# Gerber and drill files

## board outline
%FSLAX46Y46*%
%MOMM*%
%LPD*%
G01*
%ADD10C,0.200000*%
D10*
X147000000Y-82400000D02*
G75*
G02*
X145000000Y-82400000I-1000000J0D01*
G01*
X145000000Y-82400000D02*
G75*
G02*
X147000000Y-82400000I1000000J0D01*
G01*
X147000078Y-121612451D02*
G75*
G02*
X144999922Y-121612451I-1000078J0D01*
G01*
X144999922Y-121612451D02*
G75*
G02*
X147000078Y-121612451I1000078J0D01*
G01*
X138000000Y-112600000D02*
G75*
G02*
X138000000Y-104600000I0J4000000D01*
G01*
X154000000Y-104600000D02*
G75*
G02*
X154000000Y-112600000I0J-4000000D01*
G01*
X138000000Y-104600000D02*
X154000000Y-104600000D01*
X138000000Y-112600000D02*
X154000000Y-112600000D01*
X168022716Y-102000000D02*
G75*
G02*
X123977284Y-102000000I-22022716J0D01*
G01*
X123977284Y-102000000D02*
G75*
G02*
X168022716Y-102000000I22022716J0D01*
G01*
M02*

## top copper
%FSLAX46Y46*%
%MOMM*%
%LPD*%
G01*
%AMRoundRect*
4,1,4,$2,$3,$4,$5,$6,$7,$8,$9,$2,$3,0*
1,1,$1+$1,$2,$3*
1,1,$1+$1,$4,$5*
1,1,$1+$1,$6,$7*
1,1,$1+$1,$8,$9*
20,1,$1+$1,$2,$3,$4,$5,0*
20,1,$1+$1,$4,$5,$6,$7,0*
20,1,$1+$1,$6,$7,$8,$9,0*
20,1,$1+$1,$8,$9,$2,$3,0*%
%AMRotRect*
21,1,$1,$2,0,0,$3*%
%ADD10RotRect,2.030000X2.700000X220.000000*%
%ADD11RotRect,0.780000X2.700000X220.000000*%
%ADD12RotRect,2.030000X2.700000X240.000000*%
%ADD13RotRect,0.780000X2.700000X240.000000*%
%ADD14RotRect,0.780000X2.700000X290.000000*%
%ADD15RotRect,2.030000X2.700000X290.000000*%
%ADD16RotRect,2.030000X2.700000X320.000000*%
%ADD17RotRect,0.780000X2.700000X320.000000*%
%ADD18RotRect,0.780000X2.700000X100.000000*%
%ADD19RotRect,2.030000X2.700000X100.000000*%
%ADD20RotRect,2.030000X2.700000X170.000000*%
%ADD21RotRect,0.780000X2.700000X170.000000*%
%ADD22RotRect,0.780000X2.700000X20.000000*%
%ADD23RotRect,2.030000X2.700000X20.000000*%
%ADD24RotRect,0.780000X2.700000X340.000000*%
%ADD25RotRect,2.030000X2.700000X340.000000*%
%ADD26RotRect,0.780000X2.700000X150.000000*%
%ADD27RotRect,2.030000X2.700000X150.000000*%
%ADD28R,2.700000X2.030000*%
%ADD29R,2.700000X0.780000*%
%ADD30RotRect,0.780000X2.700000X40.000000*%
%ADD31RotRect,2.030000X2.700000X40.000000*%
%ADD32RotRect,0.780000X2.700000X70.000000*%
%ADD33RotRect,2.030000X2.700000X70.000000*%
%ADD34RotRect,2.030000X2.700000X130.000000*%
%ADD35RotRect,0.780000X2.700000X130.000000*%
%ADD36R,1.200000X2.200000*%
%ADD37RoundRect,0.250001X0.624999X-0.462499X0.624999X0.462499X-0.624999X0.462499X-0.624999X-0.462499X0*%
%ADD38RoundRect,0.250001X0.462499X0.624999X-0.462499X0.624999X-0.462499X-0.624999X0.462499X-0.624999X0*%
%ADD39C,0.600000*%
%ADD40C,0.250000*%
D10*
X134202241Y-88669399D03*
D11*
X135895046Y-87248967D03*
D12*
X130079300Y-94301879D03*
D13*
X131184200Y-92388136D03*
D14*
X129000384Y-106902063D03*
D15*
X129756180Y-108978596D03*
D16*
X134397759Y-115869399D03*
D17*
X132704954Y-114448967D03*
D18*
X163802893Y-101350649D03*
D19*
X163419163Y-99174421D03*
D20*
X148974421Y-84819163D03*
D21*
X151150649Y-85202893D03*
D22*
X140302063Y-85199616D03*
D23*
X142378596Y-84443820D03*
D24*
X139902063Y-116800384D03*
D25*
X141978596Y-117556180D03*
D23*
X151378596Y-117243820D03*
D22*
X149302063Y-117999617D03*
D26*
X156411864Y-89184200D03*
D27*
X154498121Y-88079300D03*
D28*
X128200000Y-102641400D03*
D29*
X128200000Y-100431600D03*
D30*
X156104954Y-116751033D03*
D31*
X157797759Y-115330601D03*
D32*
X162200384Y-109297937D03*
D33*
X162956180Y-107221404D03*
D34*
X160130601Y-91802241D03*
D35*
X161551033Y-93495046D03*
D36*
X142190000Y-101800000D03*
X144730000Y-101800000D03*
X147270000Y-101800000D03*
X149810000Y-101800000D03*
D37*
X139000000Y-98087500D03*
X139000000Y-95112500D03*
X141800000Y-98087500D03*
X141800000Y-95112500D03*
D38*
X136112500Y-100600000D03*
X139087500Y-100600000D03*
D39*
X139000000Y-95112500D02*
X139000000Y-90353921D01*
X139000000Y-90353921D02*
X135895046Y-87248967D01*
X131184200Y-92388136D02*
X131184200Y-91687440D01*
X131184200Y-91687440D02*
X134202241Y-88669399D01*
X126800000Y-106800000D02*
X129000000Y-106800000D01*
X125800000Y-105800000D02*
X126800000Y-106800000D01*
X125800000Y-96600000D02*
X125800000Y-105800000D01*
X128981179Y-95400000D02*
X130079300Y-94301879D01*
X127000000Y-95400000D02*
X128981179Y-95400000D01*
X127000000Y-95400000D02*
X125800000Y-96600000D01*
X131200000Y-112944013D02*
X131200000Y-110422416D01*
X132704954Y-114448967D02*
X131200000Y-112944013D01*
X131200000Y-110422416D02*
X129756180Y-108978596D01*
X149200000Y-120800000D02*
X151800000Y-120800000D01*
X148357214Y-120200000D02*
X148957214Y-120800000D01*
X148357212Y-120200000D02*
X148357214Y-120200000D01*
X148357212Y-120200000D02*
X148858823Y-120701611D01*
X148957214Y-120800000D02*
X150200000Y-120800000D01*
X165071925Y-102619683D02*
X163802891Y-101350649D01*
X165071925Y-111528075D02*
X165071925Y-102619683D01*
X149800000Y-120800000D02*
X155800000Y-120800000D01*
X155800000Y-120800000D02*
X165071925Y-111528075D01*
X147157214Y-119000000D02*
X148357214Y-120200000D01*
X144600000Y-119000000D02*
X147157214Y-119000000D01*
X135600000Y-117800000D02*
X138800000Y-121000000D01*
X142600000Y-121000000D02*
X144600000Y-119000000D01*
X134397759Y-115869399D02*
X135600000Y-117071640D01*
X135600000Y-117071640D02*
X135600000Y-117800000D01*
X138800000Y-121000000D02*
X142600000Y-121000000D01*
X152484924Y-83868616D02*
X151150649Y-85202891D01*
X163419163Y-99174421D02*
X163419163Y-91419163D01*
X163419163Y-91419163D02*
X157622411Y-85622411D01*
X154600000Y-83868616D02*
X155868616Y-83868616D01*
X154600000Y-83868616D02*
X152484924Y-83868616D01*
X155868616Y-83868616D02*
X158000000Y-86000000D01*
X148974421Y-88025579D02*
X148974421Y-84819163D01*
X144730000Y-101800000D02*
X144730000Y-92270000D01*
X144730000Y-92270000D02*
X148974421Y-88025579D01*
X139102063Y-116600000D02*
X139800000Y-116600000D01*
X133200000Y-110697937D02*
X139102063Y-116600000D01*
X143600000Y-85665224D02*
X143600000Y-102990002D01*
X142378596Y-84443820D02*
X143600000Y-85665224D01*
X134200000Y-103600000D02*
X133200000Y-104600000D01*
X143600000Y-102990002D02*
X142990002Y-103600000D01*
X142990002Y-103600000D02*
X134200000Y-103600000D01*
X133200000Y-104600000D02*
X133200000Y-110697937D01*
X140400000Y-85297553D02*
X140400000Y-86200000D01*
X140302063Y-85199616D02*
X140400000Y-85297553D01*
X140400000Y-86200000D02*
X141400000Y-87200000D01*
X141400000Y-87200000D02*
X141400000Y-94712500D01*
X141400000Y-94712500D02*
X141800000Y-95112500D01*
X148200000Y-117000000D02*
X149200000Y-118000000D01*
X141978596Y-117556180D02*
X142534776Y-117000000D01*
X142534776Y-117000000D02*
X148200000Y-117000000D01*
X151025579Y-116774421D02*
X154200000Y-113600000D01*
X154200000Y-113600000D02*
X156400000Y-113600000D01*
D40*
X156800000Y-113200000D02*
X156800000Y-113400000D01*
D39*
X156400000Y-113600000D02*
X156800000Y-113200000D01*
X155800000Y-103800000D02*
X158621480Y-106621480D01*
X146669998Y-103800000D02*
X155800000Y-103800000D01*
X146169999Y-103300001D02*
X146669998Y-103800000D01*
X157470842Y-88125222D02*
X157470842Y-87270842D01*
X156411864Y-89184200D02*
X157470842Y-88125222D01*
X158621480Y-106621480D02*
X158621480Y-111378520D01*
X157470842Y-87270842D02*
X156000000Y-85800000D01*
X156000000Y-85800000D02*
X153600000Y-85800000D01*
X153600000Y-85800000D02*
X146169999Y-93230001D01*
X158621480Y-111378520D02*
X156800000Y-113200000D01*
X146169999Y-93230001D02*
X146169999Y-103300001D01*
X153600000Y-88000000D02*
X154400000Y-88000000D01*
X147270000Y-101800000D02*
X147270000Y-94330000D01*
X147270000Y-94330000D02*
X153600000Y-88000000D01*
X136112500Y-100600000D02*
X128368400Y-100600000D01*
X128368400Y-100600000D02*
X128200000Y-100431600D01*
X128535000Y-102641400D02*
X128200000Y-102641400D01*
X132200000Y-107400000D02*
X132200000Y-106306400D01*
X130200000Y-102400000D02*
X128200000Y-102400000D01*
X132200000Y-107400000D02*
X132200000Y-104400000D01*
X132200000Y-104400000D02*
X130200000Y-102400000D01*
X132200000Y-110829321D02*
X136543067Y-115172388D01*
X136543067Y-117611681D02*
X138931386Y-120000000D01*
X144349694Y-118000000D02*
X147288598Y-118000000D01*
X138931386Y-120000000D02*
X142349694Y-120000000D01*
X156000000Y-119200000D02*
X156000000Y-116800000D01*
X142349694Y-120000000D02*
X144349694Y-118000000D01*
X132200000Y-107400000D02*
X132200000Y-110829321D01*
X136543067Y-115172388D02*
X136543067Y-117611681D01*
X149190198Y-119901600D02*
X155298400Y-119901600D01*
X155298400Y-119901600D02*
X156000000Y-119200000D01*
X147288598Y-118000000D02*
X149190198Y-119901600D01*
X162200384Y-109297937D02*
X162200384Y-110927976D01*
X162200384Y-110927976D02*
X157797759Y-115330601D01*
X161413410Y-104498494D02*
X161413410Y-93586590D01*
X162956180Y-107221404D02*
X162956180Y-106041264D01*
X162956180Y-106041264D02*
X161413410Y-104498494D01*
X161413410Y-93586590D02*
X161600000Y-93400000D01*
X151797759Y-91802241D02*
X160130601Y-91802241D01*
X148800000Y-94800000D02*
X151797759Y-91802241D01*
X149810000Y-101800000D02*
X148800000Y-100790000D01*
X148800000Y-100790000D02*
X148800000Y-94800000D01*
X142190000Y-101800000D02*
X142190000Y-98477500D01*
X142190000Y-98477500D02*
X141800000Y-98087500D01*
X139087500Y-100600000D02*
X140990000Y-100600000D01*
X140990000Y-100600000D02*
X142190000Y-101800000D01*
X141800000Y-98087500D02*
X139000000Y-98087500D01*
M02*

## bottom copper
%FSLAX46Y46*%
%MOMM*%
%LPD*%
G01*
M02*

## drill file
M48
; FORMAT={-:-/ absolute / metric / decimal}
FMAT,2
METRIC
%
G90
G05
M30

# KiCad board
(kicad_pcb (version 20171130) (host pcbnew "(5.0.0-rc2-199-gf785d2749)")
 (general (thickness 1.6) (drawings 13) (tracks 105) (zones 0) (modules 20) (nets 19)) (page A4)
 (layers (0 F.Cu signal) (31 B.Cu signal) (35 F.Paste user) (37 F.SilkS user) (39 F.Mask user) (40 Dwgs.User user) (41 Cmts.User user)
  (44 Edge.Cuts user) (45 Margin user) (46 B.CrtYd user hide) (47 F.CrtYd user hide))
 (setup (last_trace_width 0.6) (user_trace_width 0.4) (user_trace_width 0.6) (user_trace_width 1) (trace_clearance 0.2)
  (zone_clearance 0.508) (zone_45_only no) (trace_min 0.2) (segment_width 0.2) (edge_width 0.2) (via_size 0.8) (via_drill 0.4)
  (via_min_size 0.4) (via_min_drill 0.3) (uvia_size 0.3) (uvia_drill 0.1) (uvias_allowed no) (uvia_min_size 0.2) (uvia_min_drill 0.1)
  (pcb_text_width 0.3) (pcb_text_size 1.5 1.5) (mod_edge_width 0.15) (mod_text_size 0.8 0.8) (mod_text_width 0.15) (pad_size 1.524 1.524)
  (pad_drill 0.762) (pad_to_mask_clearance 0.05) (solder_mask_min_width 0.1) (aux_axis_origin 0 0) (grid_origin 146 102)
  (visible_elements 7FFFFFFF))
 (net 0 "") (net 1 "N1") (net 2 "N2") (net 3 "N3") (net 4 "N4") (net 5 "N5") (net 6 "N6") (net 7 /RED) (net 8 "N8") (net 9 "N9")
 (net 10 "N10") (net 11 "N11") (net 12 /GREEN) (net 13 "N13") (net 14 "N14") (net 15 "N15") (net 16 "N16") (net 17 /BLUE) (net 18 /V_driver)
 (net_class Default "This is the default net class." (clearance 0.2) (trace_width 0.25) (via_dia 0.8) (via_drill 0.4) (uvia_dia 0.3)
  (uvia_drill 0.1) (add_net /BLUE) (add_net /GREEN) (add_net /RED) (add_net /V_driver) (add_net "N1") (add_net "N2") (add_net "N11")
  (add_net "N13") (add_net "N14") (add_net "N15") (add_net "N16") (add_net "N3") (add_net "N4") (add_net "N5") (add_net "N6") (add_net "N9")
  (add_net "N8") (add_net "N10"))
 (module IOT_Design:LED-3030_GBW (layer F.Cu) (at 135 88 220)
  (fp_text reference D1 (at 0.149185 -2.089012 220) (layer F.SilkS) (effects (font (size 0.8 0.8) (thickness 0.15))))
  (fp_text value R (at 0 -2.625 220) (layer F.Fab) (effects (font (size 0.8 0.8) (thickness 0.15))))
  (pad 1 smd rect (at 1.0414 0 220) (size 2.03 2.7) (layers F.Cu F.Paste F.Mask) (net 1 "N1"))
  (pad 2 smd rect (at -1.1684 0 220) (size 0.78 2.7) (layers F.Cu F.Paste F.Mask) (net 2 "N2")))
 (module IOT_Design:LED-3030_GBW (layer F.Cu) (at 130.6 93.4 240)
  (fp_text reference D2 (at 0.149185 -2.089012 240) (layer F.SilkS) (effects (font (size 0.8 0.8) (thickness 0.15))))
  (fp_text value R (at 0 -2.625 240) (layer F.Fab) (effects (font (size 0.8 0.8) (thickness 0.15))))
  (pad 1 smd rect (at 1.0414 0 240) (size 2.03 2.7) (layers F.Cu F.Paste F.Mask) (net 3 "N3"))
  (pad 2 smd rect (at -1.1684 0 240) (size 0.78 2.7) (layers F.Cu F.Paste F.Mask) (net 1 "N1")))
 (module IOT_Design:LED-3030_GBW (layer F.Cu) (at 129.4 108 290)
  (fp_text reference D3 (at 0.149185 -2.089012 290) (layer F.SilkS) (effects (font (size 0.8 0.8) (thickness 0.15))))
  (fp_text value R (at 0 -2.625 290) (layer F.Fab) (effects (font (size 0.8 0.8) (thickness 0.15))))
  (pad 2 smd rect (at -1.1684 0 290) (size 0.78 2.7) (layers F.Cu F.Paste F.Mask) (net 3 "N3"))
  (pad 1 smd rect (at 1.0414 0 290) (size 2.03 2.7) (layers F.Cu F.Paste F.Mask) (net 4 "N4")))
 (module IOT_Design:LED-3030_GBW (layer F.Cu) (at 133.6 115.2 320)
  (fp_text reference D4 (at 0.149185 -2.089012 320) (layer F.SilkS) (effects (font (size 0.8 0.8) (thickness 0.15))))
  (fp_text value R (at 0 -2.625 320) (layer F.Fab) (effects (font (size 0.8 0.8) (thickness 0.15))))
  (pad 1 smd rect (at 1.0414 0 320) (size 2.03 2.7) (layers F.Cu F.Paste F.Mask) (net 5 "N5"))
  (pad 2 smd rect (at -1.1684 0 320) (size 0.78 2.7) (layers F.Cu F.Paste F.Mask) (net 4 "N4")))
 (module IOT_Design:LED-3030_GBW (layer F.Cu) (at 163.6 100.2 100)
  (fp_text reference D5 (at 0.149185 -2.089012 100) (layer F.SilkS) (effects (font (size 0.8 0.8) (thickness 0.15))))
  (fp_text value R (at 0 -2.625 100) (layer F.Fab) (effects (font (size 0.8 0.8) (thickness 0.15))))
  (pad 2 smd rect (at -1.1684 0.000002 100) (size 0.78 2.7) (layers F.Cu F.Paste F.Mask) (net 5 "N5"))
  (pad 1 smd rect (at 1.0414 0 100) (size 2.03 2.7) (layers F.Cu F.Paste F.Mask) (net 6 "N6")))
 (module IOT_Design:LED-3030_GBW (layer F.Cu) (at 150 85 170)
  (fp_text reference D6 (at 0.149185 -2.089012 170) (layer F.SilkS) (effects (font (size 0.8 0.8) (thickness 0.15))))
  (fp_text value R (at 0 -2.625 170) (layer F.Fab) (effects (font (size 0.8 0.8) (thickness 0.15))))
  (pad 1 smd rect (at 1.0414 0 170) (size 2.03 2.7) (layers F.Cu F.Paste F.Mask) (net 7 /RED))
  (pad 2 smd rect (at -1.1684 -0.000002 170) (size 0.78 2.7) (layers F.Cu F.Paste F.Mask) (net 6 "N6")))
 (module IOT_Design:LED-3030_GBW (layer F.Cu) (at 141.4 84.8 20)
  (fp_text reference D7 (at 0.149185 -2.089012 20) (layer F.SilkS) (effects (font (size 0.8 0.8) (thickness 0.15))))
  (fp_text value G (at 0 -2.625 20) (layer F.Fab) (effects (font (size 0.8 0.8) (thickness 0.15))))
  (pad 2 smd rect (at -1.1684 0 20) (size 0.78 2.7) (layers F.Cu F.Paste F.Mask) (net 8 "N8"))
  (pad 1 smd rect (at 1.0414 0 20) (size 2.03 2.7) (layers F.Cu F.Paste F.Mask) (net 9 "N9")))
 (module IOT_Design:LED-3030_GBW (layer F.Cu) (at 141 117.2 340)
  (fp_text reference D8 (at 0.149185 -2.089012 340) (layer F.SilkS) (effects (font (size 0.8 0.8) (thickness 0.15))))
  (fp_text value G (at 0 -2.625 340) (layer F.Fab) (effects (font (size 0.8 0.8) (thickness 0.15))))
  (pad 2 smd rect (at -1.1684 0 340) (size 0.78 2.7) (layers F.Cu F.Paste F.Mask) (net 9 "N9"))
  (pad 1 smd rect (at 1.0414 0 340) (size 2.03 2.7) (layers F.Cu F.Paste F.Mask) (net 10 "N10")))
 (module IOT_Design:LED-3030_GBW (layer F.Cu) (at 150.4 117.6 20)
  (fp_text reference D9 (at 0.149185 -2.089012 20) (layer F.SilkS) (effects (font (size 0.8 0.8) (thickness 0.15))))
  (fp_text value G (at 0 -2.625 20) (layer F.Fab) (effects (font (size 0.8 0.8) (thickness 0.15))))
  (pad 1 smd rect (at 1.0414 0 20) (size 2.03 2.7) (layers F.Cu F.Paste F.Mask) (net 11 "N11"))
  (pad 2 smd rect (at -1.1684 0.000001 20) (size 0.78 2.7) (layers F.Cu F.Paste F.Mask) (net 10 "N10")))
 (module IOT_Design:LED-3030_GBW (layer F.Cu) (at 155.4 88.6 150)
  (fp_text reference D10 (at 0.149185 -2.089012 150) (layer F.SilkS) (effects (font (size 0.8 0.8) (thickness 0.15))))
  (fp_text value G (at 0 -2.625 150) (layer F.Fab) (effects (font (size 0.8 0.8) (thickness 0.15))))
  (pad 2 smd rect (at -1.1684 0 150) (size 0.78 2.7) (layers F.Cu F.Paste F.Mask) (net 11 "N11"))
  (pad 1 smd rect (at 1.0414 0 150) (size 2.03 2.7) (layers F.Cu F.Paste F.Mask) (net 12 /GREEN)))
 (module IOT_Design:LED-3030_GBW (layer F.Cu) (at 128.2 101.6 270)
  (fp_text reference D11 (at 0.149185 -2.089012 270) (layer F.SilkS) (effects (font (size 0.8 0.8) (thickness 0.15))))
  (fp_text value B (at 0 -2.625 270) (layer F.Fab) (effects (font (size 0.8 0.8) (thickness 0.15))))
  (pad 1 smd rect (at 1.0414 0 270) (size 2.03 2.7) (layers F.Cu F.Paste F.Mask) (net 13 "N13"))
  (pad 2 smd rect (at -1.1684 0 270) (size 0.78 2.7) (layers F.Cu F.Paste F.Mask) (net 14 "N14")))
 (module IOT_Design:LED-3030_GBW (layer F.Cu) (at 157 116 40)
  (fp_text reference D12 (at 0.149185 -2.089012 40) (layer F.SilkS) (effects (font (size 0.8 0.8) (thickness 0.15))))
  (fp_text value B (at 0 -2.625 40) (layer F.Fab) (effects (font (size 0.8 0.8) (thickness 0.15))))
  (pad 2 smd rect (at -1.1684 0 40) (size 0.78 2.7) (layers F.Cu F.Paste F.Mask) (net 13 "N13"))
  (pad 1 smd rect (at 1.0414 0 40) (size 2.03 2.7) (layers F.Cu F.Paste F.Mask) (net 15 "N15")))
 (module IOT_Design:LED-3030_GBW (layer F.Cu) (at 162.6 108.2 70)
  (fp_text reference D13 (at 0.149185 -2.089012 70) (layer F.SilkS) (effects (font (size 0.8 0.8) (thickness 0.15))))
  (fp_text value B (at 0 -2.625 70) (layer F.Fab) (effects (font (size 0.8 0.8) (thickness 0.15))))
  (pad 2 smd rect (at -1.1684 0 70) (size 0.78 2.7) (layers F.Cu F.Paste F.Mask) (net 15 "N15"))
  (pad 1 smd rect (at 1.0414 0 70) (size 2.03 2.7) (layers F.Cu F.Paste F.Mask) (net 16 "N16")))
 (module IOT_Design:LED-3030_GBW (layer F.Cu) (at 160.8 92.6 130)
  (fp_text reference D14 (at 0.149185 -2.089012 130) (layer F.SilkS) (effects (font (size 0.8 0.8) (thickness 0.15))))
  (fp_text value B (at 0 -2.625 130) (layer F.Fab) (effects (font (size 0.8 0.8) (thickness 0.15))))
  (pad 1 smd rect (at 1.0414 0 130) (size 2.03 2.7) (layers F.Cu F.Paste F.Mask) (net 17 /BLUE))
  (pad 2 smd rect (at -1.1684 0 130) (size 0.78 2.7) (layers F.Cu F.Paste F.Mask) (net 16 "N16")))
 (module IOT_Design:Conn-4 (layer F.Cu) (at 146 101.8)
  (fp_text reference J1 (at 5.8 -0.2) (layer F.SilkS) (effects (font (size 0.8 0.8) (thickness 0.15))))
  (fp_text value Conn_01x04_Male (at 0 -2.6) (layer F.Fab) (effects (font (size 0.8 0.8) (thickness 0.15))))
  (pad 1 smd rect (at -3.81 0) (size 1.2 2.2) (layers F.Cu F.Paste F.Mask) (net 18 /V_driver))
  (pad 2 smd rect (at -1.27 0) (size 1.2 2.2) (layers F.Cu F.Paste F.Mask) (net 7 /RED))
  (pad 3 smd rect (at 1.27 0) (size 1.2 2.2) (layers F.Cu F.Paste F.Mask) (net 12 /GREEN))
  (pad 4 smd rect (at 3.81 0) (size 1.2 2.2) (layers F.Cu F.Paste F.Mask) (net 17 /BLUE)))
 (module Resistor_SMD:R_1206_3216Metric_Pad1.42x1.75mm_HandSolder (layer F.Cu) (at 139 96.6 90)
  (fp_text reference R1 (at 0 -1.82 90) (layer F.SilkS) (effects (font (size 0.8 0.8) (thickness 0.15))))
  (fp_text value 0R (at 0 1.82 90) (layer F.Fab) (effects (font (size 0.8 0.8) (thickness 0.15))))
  (pad 1 smd roundrect (at -1.4875 0 90) (size 1.425 1.75) (layers F.Cu F.Paste F.Mask) (roundrect_rratio 0.175439) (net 18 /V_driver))
  (pad 2 smd roundrect (at 1.4875 0 90) (size 1.425 1.75) (layers F.Cu F.Paste F.Mask) (roundrect_rratio 0.175439) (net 2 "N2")))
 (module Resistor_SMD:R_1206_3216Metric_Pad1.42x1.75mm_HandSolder (layer F.Cu) (at 141.8 96.6 90)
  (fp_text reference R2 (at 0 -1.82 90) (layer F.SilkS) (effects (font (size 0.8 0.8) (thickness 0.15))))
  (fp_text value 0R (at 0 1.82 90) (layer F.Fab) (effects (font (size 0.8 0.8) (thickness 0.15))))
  (pad 1 smd roundrect (at -1.4875 0 90) (size 1.425 1.75) (layers F.Cu F.Paste F.Mask) (roundrect_rratio 0.175439) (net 18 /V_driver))
  (pad 2 smd roundrect (at 1.4875 0 90) (size 1.425 1.75) (layers F.Cu F.Paste F.Mask) (roundrect_rratio 0.175439) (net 8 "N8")))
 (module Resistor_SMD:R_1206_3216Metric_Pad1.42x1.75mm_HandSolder (layer F.Cu) (at 137.6 100.6 180)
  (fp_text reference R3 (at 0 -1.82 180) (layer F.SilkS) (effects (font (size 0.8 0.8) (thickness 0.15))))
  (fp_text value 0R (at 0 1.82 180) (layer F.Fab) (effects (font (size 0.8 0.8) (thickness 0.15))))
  (pad 2 smd roundrect (at 1.4875 0 180) (size 1.425 1.75) (layers F.Cu F.Paste F.Mask) (roundrect_rratio 0.175439) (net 14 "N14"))
  (pad 1 smd roundrect (at -1.4875 0 180) (size 1.425 1.75) (layers F.Cu F.Paste F.Mask) (roundrect_rratio 0.175439) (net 18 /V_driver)))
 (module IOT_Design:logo (layer F.Cu) (at 176.6 110.2)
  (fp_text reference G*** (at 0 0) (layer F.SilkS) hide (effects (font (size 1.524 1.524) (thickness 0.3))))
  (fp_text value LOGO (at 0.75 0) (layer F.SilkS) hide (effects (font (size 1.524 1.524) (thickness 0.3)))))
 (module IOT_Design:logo (layer F.Cu) (at 146 92)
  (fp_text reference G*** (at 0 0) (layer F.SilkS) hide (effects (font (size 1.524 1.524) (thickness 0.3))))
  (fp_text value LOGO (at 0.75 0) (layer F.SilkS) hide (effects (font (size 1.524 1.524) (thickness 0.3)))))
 (gr_circle (center 146 82.4) (end 147 82.4) (layer Edge.Cuts) (width 0.2))
 (gr_circle (center 146 121.612451) (end 147 121.6) (layer Edge.Cuts) (width 0.2))
 (gr_arc (start 138 108.6) (end 138 104.6) (angle -180) (layer Edge.Cuts) (width 0.2))
 (gr_arc (start 154 108.6) (end 154 112.6) (angle -180) (layer Edge.Cuts) (width 0.2))
 (gr_line (start 138 104.6) (end 154 104.6) (layer Edge.Cuts) (width 0.2))
 (gr_line (start 138 112.6) (end 154 112.6) (layer Edge.Cuts) (width 0.2))
 (gr_circle (center 146 102) (end 168.022716 102) (layer Edge.Cuts) (width 0.2))
 (segment (start 139 95.1125) (end 139 90.353921) (width 0.6) (layer F.Cu) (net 2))
 (segment (start 139 90.353921) (end 135.895046 87.248967) (width 0.6) (layer F.Cu) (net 2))
 (segment (start 131.1842 92.388136) (end 131.1842 91.68744) (width 0.6) (layer F.Cu) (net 1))
 (segment (start 131.1842 91.68744) (end 134.202241 88.669399) (width 0.6) (layer F.Cu) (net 1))
 (segment (start 126.8 106.8) (end 129 106.8) (width 0.6) (layer F.Cu) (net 3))
 (segment (start 125.8 105.8) (end 126.8 106.8) (width 0.6) (layer F.Cu) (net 3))
 (segment (start 125.8 96.6) (end 125.8 105.8) (width 0.6) (layer F.Cu) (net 3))
 (segment (start 128.981179 95.4) (end 130.0793 94.301879) (width 0.6) (layer F.Cu) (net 3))
 (segment (start 127 95.4) (end 128.981179 95.4) (width 0.6) (layer F.Cu) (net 3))
 (segment (start 127 95.4) (end 125.8 96.6) (width 0.6) (layer F.Cu) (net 3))
 (segment (start 131.2 112.944013) (end 131.2 110.422416) (width 0.6) (layer F.Cu) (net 4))
 (segment (start 132.704954 114.448967) (end 131.2 112.944013) (width 0.6) (layer F.Cu) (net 4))
 (segment (start 131.2 110.422416) (end 129.75618 108.978596) (width 0.6) (layer F.Cu) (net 4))
 (segment (start 149.2 120.8) (end 151.8 120.8) (width 0.6) (layer F.Cu) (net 5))
 (segment (start 148.357214 120.2) (end 148.957214 120.8) (width 0.6) (layer F.Cu) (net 5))
 (segment (start 148.357212 120.2) (end 148.357214 120.2) (width 0.6) (layer F.Cu) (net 5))
 (segment (start 148.357212 120.2) (end 148.858823 120.701611) (width 0.6) (layer F.Cu) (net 5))
 (segment (start 148.957214 120.8) (end 150.2 120.8) (width 0.6) (layer F.Cu) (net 5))
 (segment (start 165.071925 102.619683) (end 163.802891 101.350649) (width 0.6) (layer F.Cu) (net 5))
 (segment (start 165.071925 111.528075) (end 165.071925 102.619683) (width 0.6) (layer F.Cu) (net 5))
 (segment (start 149.8 120.8) (end 155.8 120.8) (width 0.6) (layer F.Cu) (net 5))
 (segment (start 155.8 120.8) (end 165.071925 111.528075) (width 0.6) (layer F.Cu) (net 5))
 (segment (start 147.157214 119) (end 148.357214 120.2) (width 0.6) (layer F.Cu) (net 5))
 (segment (start 144.6 119) (end 147.157214 119) (width 0.6) (layer F.Cu) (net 5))
 (segment (start 135.6 117.8) (end 138.8 121) (width 0.6) (layer F.Cu) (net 5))
 (segment (start 142.6 121) (end 144.6 119) (width 0.6) (layer F.Cu) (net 5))
 (segment (start 134.397759 115.869399) (end 135.6 117.07164) (width 0.6) (layer F.Cu) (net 5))
 (segment (start 135.6 117.07164) (end 135.6 117.8) (width 0.6) (layer F.Cu) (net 5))
 (segment (start 138.8 121) (end 142.6 121) (width 0.6) (layer F.Cu) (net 5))
 (segment (start 152.484924 83.868616) (end 151.150649 85.202891) (width 0.6) (layer F.Cu) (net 6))
 (segment (start 163.419163 99.174421) (end 163.419163 91.419163) (width 0.6) (layer F.Cu) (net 6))
 (segment (start 163.419163 91.419163) (end 157.622411 85.622411) (width 0.6) (layer F.Cu) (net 6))
 (segment (start 154.6 83.868616) (end 155.868616 83.868616) (width 0.6) (layer F.Cu) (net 6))
 (segment (start 154.6 83.868616) (end 152.484924 83.868616) (width 0.6) (layer F.Cu) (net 6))
 (segment (start 155.868616 83.868616) (end 158 86) (width 0.6) (layer F.Cu) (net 6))
 (segment (start 148.974421 88.025579) (end 148.974421 84.819163) (width 0.6) (layer F.Cu) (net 7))
 (segment (start 144.73 101.8) (end 144.73 92.27) (width 0.6) (layer F.Cu) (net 7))
 (segment (start 144.73 92.27) (end 148.974421 88.025579) (width 0.6) (layer F.Cu) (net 7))
 (segment (start 139.102063 116.6) (end 139.8 116.6) (width 0.6) (layer F.Cu) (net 9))
 (segment (start 133.2 110.697937) (end 139.102063 116.6) (width 0.6) (layer F.Cu) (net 9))
 (segment (start 143.6 85.665224) (end 143.6 102.990002) (width 0.6) (layer F.Cu) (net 9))
 (segment (start 142.378596 84.44382) (end 143.6 85.665224) (width 0.6) (layer F.Cu) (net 9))
 (segment (start 134.2 103.6) (end 133.2 104.6) (width 0.6) (layer F.Cu) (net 9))
 (segment (start 143.6 102.990002) (end 142.990002 103.6) (width 0.6) (layer F.Cu) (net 9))
 (segment (start 142.990002 103.6) (end 134.2 103.6) (width 0.6) (layer F.Cu) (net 9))
 (segment (start 133.2 104.6) (end 133.2 110.697937) (width 0.6) (layer F.Cu) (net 9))
 (segment (start 140.4 85.297553) (end 140.4 86.2) (width 0.6) (layer F.Cu) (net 8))
 (segment (start 140.302063 85.199616) (end 140.4 85.297553) (width 0.6) (layer F.Cu) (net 8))
 (segment (start 140.4 86.2) (end 141.4 87.2) (width 0.6) (layer F.Cu) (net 8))
 (segment (start 141.4 87.2) (end 141.4 94.7125) (width 0.6) (layer F.Cu) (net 8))
 (segment (start 141.4 94.7125) (end 141.8 95.1125) (width 0.6) (layer F.Cu) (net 8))
 (segment (start 148.2 117) (end 149.2 118) (width 0.6) (layer F.Cu) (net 10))
 (segment (start 141.978596 117.55618) (end 142.534776 117) (width 0.6) (layer F.Cu) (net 10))
 (segment (start 142.534776 117) (end 148.2 117) (width 0.6) (layer F.Cu) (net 10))
 (segment (start 151.025579 116.774421) (end 154.2 113.6) (width 0.6) (layer F.Cu) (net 11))
 (segment (start 154.2 113.6) (end 156.4 113.6) (width 0.6) (layer F.Cu) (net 11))
 (segment (start 156.8 113.2) (end 156.8 113.4) (width 0.25) (layer F.Cu) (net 11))
 (segment (start 156.4 113.6) (end 156.8 113.2) (width 0.6) (layer F.Cu) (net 11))
 (segment (start 155.8 103.8) (end 158.62148 106.62148) (width 0.6) (layer F.Cu) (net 11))
 (segment (start 146.669998 103.8) (end 155.8 103.8) (width 0.6) (layer F.Cu) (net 11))
 (segment (start 146.169999 103.300001) (end 146.669998 103.8) (width 0.6) (layer F.Cu) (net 11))
 (segment (start 157.470842 88.125222) (end 157.470842 87.270842) (width 0.6) (layer F.Cu) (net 11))
 (segment (start 156.411864 89.1842) (end 157.470842 88.125222) (width 0.6) (layer F.Cu) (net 11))
 (segment (start 158.62148 106.62148) (end 158.62148 111.37852) (width 0.6) (layer F.Cu) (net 11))
 (segment (start 157.470842 87.270842) (end 156 85.8) (width 0.6) (layer F.Cu) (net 11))
 (segment (start 156 85.8) (end 153.6 85.8) (width 0.6) (layer F.Cu) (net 11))
 (segment (start 153.6 85.8) (end 146.169999 93.230001) (width 0.6) (layer F.Cu) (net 11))
 (segment (start 158.62148 111.37852) (end 156.8 113.2) (width 0.6) (layer F.Cu) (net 11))
 (segment (start 146.169999 93.230001) (end 146.169999 103.300001) (width 0.6) (layer F.Cu) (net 11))
 (segment (start 153.6 88) (end 154.4 88) (width 0.6) (layer F.Cu) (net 12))
 (segment (start 147.27 101.8) (end 147.27 94.33) (width 0.6) (layer F.Cu) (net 12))
 (segment (start 147.27 94.33) (end 153.6 88) (width 0.6) (layer F.Cu) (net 12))
 (segment (start 136.1125 100.6) (end 128.3684 100.6) (width 0.6) (layer F.Cu) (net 14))
 (segment (start 128.3684 100.6) (end 128.2 100.4316) (width 0.6) (layer F.Cu) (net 14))
 (segment (start 128.535 102.6414) (end 128.2 102.6414) (width 0.6) (layer F.Cu) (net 13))
 (segment (start 132.2 107.4) (end 132.2 106.3064) (width 0.6) (layer F.Cu) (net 13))
 (segment (start 130.2 102.4) (end 128.2 102.4) (width 0.6) (layer F.Cu) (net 13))
 (segment (start 132.2 107.4) (end 132.2 104.4) (width 0.6) (layer F.Cu) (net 13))
 (segment (start 132.2 104.4) (end 130.2 102.4) (width 0.6) (layer F.Cu) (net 13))
 (segment (start 132.2 110.829321) (end 136.543067 115.172388) (width 0.6) (layer F.Cu) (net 13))
 (segment (start 136.543067 117.611681) (end 138.931386 120) (width 0.6) (layer F.Cu) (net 13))
 (segment (start 144.349694 118) (end 147.288598 118) (width 0.6) (layer F.Cu) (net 13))
 (segment (start 138.931386 120) (end 142.349694 120) (width 0.6) (layer F.Cu) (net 13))
 (segment (start 156 119.2) (end 156 116.8) (width 0.6) (layer F.Cu) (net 13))
 (segment (start 142.349694 120) (end 144.349694 118) (width 0.6) (layer F.Cu) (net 13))
 (segment (start 132.2 107.4) (end 132.2 110.829321) (width 0.6) (layer F.Cu) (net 13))
 (segment (start 136.543067 115.172388) (end 136.543067 117.611681) (width 0.6) (layer F.Cu) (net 13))
 (segment (start 149.190198 119.9016) (end 155.2984 119.9016) (width 0.6) (layer F.Cu) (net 13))
 (segment (start 155.2984 119.9016) (end 156 119.2) (width 0.6) (layer F.Cu) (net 13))
 (segment (start 147.288598 118) (end 149.190198 119.9016) (width 0.6) (layer F.Cu) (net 13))
 (segment (start 162.200384 109.297937) (end 162.200384 110.927976) (width 0.6) (layer F.Cu) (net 15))
 (segment (start 162.200384 110.927976) (end 157.797759 115.330601) (width 0.6) (layer F.Cu) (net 15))
 (segment (start 161.41341 104.498494) (end 161.41341 93.58659) (width 0.6) (layer F.Cu) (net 16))
 (segment (start 162.95618 107.221404) (end 162.95618 106.041264) (width 0.6) (layer F.Cu) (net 16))
 (segment (start 162.95618 106.041264) (end 161.41341 104.498494) (width 0.6) (layer F.Cu) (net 16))
 (segment (start 161.41341 93.58659) (end 161.6 93.4) (width 0.6) (layer F.Cu) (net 16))
 (segment (start 151.797759 91.802241) (end 160.130601 91.802241) (width 0.6) (layer F.Cu) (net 17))
 (segment (start 148.8 94.8) (end 151.797759 91.802241) (width 0.6) (layer F.Cu) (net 17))
 (segment (start 149.81 101.8) (end 148.8 100.79) (width 0.6) (layer F.Cu) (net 17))
 (segment (start 148.8 100.79) (end 148.8 94.8) (width 0.6) (layer F.Cu) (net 17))
 (segment (start 142.19 101.8) (end 142.19 98.4775) (width 0.6) (layer F.Cu) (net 18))
 (segment (start 142.19 98.4775) (end 141.8 98.0875) (width 0.6) (layer F.Cu) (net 18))
 (segment (start 139.0875 100.6) (end 140.99 100.6) (width 0.6) (layer F.Cu) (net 18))
 (segment (start 140.99 100.6) (end 142.19 101.8) (width 0.6) (layer F.Cu) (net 18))
 (segment (start 141.8 98.0875) (end 139 98.0875) (width 0.6) (layer F.Cu) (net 18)))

